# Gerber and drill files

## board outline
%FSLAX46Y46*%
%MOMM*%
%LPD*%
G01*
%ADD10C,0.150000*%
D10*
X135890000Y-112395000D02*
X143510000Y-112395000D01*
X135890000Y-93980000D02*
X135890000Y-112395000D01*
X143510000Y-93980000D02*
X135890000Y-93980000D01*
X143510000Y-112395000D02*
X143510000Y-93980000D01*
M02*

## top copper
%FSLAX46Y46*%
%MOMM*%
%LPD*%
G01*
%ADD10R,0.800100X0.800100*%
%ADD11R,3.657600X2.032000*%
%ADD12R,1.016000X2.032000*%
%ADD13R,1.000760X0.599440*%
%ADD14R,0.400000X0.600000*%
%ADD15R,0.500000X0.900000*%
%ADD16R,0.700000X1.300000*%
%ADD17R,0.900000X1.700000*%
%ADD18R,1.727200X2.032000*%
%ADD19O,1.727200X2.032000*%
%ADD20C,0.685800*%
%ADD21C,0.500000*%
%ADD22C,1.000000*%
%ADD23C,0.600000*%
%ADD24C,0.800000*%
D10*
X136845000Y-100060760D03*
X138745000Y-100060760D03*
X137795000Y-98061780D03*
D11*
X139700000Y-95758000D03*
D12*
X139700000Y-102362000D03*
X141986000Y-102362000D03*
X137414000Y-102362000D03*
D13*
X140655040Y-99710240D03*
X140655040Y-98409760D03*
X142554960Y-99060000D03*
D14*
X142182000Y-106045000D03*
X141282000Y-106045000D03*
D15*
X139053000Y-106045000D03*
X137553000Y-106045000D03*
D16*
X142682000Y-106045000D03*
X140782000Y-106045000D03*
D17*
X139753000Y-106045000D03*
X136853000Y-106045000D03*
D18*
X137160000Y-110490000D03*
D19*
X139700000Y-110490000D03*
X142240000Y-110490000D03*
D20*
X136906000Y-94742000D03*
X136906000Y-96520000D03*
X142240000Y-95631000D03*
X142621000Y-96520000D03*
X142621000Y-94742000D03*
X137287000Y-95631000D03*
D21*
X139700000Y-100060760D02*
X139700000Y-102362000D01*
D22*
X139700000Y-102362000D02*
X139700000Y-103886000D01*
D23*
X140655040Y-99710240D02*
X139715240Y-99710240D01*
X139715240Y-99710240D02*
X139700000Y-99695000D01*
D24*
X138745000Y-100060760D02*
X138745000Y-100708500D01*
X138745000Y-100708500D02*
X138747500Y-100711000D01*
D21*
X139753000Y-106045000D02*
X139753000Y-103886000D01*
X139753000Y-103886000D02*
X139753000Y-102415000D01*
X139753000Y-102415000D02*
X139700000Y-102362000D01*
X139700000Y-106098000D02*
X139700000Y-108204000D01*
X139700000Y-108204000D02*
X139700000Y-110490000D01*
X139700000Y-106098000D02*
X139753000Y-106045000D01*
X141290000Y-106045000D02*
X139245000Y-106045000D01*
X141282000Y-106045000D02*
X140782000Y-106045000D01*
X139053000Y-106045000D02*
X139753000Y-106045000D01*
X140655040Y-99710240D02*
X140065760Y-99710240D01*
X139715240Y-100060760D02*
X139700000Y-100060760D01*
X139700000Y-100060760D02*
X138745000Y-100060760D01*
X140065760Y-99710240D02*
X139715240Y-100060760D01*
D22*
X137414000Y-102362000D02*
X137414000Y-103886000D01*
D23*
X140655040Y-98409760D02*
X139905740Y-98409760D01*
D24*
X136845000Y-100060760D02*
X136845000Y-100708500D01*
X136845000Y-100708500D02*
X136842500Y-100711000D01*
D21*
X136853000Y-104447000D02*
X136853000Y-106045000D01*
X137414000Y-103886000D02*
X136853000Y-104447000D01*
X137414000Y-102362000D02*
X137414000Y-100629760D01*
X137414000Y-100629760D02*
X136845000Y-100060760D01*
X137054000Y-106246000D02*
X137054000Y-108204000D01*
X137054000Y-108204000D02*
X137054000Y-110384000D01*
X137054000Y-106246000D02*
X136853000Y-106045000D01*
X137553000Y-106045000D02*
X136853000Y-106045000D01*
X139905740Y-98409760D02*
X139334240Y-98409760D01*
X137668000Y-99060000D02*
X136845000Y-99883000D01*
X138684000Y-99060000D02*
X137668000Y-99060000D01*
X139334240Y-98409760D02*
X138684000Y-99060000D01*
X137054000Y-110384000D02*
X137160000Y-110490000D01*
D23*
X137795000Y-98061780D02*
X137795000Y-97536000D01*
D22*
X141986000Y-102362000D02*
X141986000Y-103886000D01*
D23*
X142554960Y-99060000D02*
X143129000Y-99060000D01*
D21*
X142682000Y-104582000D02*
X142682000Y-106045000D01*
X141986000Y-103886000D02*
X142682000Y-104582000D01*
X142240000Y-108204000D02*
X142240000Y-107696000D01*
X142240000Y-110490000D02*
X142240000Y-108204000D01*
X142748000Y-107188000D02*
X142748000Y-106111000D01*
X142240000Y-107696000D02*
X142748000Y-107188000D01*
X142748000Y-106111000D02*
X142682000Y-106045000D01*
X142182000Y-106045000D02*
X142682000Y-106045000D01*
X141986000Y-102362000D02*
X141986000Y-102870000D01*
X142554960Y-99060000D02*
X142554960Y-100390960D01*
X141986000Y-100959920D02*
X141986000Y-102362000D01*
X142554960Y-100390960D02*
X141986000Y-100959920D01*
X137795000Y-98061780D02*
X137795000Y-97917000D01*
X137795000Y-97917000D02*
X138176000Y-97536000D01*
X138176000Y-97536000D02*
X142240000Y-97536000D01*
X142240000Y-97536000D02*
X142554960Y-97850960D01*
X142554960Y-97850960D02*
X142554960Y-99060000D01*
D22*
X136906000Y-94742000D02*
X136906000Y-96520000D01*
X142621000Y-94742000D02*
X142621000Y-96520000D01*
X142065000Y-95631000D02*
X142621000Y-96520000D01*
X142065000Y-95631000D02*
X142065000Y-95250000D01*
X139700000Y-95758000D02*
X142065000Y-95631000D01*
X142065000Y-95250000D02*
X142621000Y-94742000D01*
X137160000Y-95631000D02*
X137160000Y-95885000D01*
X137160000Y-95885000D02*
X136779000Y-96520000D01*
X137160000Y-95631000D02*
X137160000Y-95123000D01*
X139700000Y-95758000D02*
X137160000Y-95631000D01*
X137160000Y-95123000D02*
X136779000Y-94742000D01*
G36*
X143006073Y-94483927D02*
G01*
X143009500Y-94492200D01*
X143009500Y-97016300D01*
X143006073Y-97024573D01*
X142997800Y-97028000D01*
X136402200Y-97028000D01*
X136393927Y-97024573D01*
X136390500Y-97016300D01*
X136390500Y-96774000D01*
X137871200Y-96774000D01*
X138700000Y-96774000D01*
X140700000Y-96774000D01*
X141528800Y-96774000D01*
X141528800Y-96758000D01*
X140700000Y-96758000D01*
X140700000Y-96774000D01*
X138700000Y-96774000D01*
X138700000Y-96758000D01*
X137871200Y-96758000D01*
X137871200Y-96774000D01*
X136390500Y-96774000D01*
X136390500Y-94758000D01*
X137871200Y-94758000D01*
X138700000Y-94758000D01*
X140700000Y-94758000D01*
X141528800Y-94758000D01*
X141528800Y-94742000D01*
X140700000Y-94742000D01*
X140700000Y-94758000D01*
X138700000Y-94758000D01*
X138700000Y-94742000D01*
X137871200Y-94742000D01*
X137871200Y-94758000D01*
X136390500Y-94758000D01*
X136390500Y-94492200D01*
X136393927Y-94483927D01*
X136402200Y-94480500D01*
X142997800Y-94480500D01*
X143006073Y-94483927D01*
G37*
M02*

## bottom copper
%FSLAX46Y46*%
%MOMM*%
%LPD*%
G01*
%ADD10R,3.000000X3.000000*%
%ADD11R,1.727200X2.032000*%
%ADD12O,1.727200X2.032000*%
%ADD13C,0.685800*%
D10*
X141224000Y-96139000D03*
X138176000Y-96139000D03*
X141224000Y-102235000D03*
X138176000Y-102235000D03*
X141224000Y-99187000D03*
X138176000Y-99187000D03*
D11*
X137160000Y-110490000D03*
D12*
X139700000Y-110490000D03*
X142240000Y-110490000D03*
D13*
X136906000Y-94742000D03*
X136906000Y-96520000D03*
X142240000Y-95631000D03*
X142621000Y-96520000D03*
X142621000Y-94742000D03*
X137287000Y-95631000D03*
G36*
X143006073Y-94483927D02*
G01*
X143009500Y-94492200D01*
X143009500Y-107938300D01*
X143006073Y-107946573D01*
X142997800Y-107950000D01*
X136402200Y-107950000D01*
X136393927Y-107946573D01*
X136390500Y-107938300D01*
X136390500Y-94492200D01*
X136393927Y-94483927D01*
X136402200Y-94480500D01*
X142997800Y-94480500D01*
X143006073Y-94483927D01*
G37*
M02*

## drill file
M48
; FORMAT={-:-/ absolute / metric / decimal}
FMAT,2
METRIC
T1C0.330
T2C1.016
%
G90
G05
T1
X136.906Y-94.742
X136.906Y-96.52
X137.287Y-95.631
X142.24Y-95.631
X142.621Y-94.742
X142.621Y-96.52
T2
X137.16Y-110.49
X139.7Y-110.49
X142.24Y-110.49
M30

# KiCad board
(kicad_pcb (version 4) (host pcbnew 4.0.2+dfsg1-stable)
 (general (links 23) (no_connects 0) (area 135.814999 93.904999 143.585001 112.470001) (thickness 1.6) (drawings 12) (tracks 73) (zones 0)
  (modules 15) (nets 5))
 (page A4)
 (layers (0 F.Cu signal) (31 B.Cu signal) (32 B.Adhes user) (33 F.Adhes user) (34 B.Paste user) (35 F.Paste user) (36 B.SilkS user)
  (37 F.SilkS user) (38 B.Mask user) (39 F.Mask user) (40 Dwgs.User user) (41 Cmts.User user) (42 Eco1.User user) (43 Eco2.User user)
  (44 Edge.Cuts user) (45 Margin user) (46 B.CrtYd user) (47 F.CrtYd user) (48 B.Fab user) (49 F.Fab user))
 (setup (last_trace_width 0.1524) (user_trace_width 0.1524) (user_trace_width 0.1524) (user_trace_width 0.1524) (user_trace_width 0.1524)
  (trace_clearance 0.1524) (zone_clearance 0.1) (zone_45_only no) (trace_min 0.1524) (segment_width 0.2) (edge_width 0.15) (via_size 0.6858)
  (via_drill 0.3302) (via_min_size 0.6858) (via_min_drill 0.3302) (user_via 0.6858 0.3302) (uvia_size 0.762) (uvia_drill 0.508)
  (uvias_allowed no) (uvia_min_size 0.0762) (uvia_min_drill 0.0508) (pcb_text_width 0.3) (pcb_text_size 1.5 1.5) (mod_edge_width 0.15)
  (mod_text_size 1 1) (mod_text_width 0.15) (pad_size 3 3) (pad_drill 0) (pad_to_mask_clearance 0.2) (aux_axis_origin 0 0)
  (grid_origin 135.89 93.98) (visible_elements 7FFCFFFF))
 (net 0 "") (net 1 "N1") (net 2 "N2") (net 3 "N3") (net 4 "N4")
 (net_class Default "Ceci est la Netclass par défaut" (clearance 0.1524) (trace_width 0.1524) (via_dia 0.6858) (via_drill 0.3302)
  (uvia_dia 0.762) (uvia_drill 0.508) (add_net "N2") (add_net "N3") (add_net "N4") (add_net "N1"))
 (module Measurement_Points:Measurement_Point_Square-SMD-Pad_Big (layer B.Cu) (at 141.224 96.139)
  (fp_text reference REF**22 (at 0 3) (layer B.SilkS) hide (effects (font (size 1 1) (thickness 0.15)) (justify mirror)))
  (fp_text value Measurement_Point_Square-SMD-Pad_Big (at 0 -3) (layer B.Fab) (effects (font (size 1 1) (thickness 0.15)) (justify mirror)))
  (pad 1 smd rect (at 0 0) (size 3 3) (layers B.Cu B.Mask) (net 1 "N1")))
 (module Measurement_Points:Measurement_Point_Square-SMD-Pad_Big (layer B.Cu) (at 138.176 96.139)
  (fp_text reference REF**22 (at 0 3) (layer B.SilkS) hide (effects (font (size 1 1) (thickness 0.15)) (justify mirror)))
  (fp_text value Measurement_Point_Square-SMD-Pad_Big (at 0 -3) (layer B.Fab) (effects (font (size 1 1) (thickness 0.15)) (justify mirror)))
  (pad 1 smd rect (at 0 0) (size 3 3) (layers B.Cu B.Mask) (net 1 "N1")))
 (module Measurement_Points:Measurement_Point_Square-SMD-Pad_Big (layer B.Cu) (at 141.224 102.235)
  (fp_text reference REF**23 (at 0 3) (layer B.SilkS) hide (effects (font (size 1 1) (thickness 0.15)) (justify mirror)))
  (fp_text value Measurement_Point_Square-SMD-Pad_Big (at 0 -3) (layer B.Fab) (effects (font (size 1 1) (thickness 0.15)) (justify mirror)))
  (pad 1 smd rect (at 0 0) (size 3 3) (layers B.Cu B.Mask) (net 1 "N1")))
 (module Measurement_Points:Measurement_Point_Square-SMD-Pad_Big (layer B.Cu) (at 138.176 102.235)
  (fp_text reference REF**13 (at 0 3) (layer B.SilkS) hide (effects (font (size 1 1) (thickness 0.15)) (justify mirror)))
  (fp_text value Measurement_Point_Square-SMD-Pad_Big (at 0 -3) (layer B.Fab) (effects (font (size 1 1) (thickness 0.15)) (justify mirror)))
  (pad 1 smd rect (at 0 0) (size 3 3) (layers B.Cu B.Mask) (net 1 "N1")))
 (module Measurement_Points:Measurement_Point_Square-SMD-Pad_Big (layer B.Cu) (at 141.224 99.187)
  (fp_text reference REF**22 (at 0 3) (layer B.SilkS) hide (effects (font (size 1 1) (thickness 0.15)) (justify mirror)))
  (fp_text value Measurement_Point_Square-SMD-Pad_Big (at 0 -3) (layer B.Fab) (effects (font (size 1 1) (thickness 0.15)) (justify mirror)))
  (pad 1 smd rect (at 0 0) (size 3 3) (layers B.Cu B.Mask) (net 1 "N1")))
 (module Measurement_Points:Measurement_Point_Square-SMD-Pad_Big (layer B.Cu) (at 138.176 99.187) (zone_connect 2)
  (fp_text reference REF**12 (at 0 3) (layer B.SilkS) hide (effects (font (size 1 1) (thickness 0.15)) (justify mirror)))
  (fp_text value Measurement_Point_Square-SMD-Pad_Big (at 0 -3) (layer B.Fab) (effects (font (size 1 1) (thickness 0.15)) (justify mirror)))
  (pad 1 smd rect (at 0 0) (size 3 3) (layers B.Cu B.Mask) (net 1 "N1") (zone_connect 2)))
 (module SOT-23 (layer F.Cu) (at 137.795 99.06)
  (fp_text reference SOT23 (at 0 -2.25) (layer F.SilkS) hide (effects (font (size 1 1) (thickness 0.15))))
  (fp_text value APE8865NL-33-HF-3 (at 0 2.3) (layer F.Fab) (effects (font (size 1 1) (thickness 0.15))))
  (pad 1 smd rect (at -0.95 1.00076) (size 0.8001 0.8001) (layers F.Cu F.Paste F.Mask) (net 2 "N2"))
  (pad 2 smd rect (at 0.95 1.00076) (size 0.8001 0.8001) (layers F.Cu F.Paste F.Mask) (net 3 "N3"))
  (pad 3 smd rect (at 0 -0.99822) (size 0.8001 0.8001) (layers F.Cu F.Paste F.Mask) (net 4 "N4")))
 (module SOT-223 (layer F.Cu) (at 139.7 99.06)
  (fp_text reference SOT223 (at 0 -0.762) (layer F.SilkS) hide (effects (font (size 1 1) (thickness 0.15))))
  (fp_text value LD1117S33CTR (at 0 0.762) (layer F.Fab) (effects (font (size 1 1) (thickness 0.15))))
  (pad 4 smd rect (at 0 -3.302) (size 3.6576 2.032) (layers F.Cu F.Paste F.Mask) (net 1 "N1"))
  (pad 2 smd rect (at 0 3.302) (size 1.016 2.032) (layers F.Cu F.Paste F.Mask) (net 3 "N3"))
  (pad 3 smd rect (at 2.286 3.302) (size 1.016 2.032) (layers F.Cu F.Paste F.Mask) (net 4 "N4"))
  (pad 1 smd rect (at -2.286 3.302) (size 1.016 2.032) (layers F.Cu F.Paste F.Mask) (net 2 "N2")))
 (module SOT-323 (layer F.Cu) (at 141.605 99.06 90)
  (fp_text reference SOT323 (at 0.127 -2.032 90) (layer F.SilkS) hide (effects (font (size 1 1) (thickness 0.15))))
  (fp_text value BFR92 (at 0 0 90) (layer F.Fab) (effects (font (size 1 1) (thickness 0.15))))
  (pad 2 smd rect (at -0.65024 -0.94996 90) (size 0.59944 1.00076) (layers F.Cu F.Paste F.Mask) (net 3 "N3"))
  (pad 1 smd rect (at 0.65024 -0.94996 90) (size 0.59944 1.00076) (layers F.Cu F.Paste F.Mask) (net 2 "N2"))
  (pad 3 smd rect (at 0 0.94996 90) (size 0.59944 1.00076) (layers F.Cu F.Paste F.Mask) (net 4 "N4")))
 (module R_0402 (layer F.Cu) (at 141.732 106.045 180)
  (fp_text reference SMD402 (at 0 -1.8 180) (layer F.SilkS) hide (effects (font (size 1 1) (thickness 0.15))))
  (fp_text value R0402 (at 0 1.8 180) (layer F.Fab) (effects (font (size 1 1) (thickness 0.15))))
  (pad 1 smd rect (at -0.45 0 180) (size 0.4 0.6) (layers F.Cu F.Paste F.Mask) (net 4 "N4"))
  (pad 2 smd rect (at 0.45 0 180) (size 0.4 0.6) (layers F.Cu F.Paste F.Mask) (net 3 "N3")))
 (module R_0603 (layer F.Cu) (at 138.303 106.045 180)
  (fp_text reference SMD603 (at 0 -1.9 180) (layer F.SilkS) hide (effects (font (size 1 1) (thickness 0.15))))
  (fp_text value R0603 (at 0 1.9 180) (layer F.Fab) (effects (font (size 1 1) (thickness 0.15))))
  (pad 1 smd rect (at -0.75 0 180) (size 0.5 0.9) (layers F.Cu F.Paste F.Mask) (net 3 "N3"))
  (pad 2 smd rect (at 0.75 0 180) (size 0.5 0.9) (layers F.Cu F.Paste F.Mask) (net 2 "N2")))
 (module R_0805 (layer F.Cu) (at 141.732 106.045 180)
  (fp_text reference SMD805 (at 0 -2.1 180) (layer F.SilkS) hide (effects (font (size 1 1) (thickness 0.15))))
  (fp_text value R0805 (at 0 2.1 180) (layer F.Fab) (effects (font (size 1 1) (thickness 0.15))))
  (pad 1 smd rect (at -0.95 0 180) (size 0.7 1.3) (layers F.Cu F.Paste F.Mask) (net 4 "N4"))
  (pad 2 smd rect (at 0.95 0 180) (size 0.7 1.3) (layers F.Cu F.Paste F.Mask) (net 3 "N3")))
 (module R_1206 (layer F.Cu) (at 138.303 106.045 180)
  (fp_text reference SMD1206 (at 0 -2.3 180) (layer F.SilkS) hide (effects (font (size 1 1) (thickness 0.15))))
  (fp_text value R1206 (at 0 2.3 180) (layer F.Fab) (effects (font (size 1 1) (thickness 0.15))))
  (pad 1 smd rect (at -1.45 0 180) (size 0.9 1.7) (layers F.Cu F.Paste F.Mask) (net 3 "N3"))
  (pad 2 smd rect (at 1.45 0 180) (size 0.9 1.7) (layers F.Cu F.Paste F.Mask) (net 2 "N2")))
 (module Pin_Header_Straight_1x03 (layer F.Cu) (at 137.16 110.49 90)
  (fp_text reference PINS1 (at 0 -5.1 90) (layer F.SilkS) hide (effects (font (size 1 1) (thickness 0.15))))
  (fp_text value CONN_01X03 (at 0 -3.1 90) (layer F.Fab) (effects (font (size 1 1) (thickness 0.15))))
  (pad 1 thru_hole rect (at 0 0 90) (size 2.032 1.7272) (drill 1.016) (layers *.Cu *.Mask F.SilkS) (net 2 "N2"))
  (pad 2 thru_hole oval (at 0 2.54 90) (size 2.032 1.7272) (drill 1.016) (layers *.Cu *.Mask F.SilkS) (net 3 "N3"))
  (pad 3 thru_hole oval (at 0 5.08 90) (size 2.032 1.7272) (drill 1.016) (layers *.Cu *.Mask F.SilkS) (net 4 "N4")))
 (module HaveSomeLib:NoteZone (layer B.Cu) (at 139.7 108.204)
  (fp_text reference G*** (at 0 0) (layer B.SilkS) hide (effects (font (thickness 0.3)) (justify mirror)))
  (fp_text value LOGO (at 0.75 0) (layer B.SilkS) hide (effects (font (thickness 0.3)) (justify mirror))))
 (gr_line (start 135.89 112.395) (end 143.51 112.395) (angle 90) (layer Edge.Cuts) (width 0.15))
 (gr_line (start 135.89 93.98) (end 135.89 112.395) (angle 90) (layer Edge.Cuts) (width 0.15))
 (gr_line (start 143.51 93.98) (end 135.89 93.98) (angle 90) (layer Edge.Cuts) (width 0.15))
 (gr_line (start 143.51 112.395) (end 143.51 93.98) (angle 90) (layer Edge.Cuts) (width 0.15))
 (segment (start 139.7 100.06076) (end 139.7 102.362) (width 0.5) (layer F.Cu) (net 3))
 (segment (start 139.7 102.362) (end 139.7 103.886) (width 1) (layer F.Cu) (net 3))
 (segment (start 140.65504 99.71024) (end 139.71524 99.71024) (width 0.6) (layer F.Cu) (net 3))
 (segment (start 139.71524 99.71024) (end 139.7 99.695) (width 0.6) (layer F.Cu) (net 3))
 (segment (start 138.745 100.06076) (end 138.745 100.7085) (width 0.8) (layer F.Cu) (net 3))
 (segment (start 138.745 100.7085) (end 138.7475 100.711) (width 0.8) (layer F.Cu) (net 3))
 (segment (start 139.753 106.045) (end 139.753 103.886) (width 0.5) (layer F.Cu) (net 3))
 (segment (start 139.753 103.886) (end 139.753 102.415) (width 0.5) (layer F.Cu) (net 3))
 (segment (start 139.753 102.415) (end 139.7 102.362) (width 0.5) (layer F.Cu) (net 3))
 (segment (start 139.7 106.098) (end 139.7 108.204) (width 0.5) (layer F.Cu) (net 3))
 (segment (start 139.7 108.204) (end 139.7 110.49) (width 0.5) (layer F.Cu) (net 3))
 (segment (start 139.7 106.098) (end 139.753 106.045) (width 0.5) (layer F.Cu) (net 3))
 (segment (start 141.29 106.045) (end 139.245 106.045) (width 0.5) (layer F.Cu) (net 3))
 (segment (start 141.282 106.045) (end 140.782 106.045) (width 0.5) (layer F.Cu) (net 3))
 (segment (start 139.053 106.045) (end 139.753 106.045) (width 0.5) (layer F.Cu) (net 3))
 (segment (start 140.65504 99.71024) (end 140.06576 99.71024) (width 0.5) (layer F.Cu) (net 3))
 (segment (start 139.71524 100.06076) (end 139.7 100.06076) (width 0.5) (layer F.Cu) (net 3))
 (segment (start 139.7 100.06076) (end 138.745 100.06076) (width 0.5) (layer F.Cu) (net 3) (status 20))
 (segment (start 140.06576 99.71024) (end 139.71524 100.06076) (width 0.5) (layer F.Cu) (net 3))
 (segment (start 137.414 102.362) (end 137.414 103.886) (width 1) (layer F.Cu) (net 2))
 (segment (start 140.65504 98.40976) (end 139.90574 98.40976) (width 0.6) (layer F.Cu) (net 2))
 (segment (start 136.845 100.06076) (end 136.845 100.7085) (width 0.8) (layer F.Cu) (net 2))
 (segment (start 136.845 100.7085) (end 136.8425 100.711) (width 0.8) (layer F.Cu) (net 2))
 (segment (start 136.853 104.447) (end 136.853 106.045) (width 0.5) (layer F.Cu) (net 2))
 (segment (start 137.414 103.886) (end 136.853 104.447) (width 0.5) (layer F.Cu) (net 2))
 (segment (start 137.414 102.362) (end 137.414 100.62976) (width 0.5) (layer F.Cu) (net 2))
 (segment (start 137.414 100.62976) (end 136.845 100.06076) (width 0.5) (layer F.Cu) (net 2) (status 20))
 (segment (start 137.054 106.246) (end 137.054 108.204) (width 0.5) (layer F.Cu) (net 2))
 (segment (start 137.054 108.204) (end 137.054 110.384) (width 0.5) (layer F.Cu) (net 2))
 (segment (start 137.054 106.246) (end 136.853 106.045) (width 0.5) (layer F.Cu) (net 2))
 (segment (start 137.553 106.045) (end 136.853 106.045) (width 0.5) (layer F.Cu) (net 2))
 (segment (start 139.90574 98.40976) (end 139.33424 98.40976) (width 0.5) (layer F.Cu) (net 2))
 (segment (start 137.668 99.06) (end 136.845 99.883) (width 0.5) (layer F.Cu) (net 2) (status 20))
 (segment (start 138.684 99.06) (end 137.668 99.06) (width 0.5) (layer F.Cu) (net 2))
 (segment (start 139.33424 98.40976) (end 138.684 99.06) (width 0.5) (layer F.Cu) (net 2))
 (segment (start 137.054 110.384) (end 137.16 110.49) (width 0.5) (layer F.Cu) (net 2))
 (segment (start 137.795 98.06178) (end 137.795 97.536) (width 0.6) (layer F.Cu) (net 4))
 (segment (start 141.986 102.362) (end 141.986 103.886) (width 1) (layer F.Cu) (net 4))
 (segment (start 142.55496 99.06) (end 143.129 99.06) (width 0.6) (layer F.Cu) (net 4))
 (segment (start 142.682 104.582) (end 142.682 106.045) (width 0.5) (layer F.Cu) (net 4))
 (segment (start 141.986 103.886) (end 142.682 104.582) (width 0.5) (layer F.Cu) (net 4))
 (segment (start 142.24 108.204) (end 142.24 107.696) (width 0.5) (layer F.Cu) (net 4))
 (segment (start 142.24 110.49) (end 142.24 108.204) (width 0.5) (layer F.Cu) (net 4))
 (segment (start 142.748 107.188) (end 142.748 106.111) (width 0.5) (layer F.Cu) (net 4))
 (segment (start 142.24 107.696) (end 142.748 107.188) (width 0.5) (layer F.Cu) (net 4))
 (segment (start 142.748 106.111) (end 142.682 106.045) (width 0.5) (layer F.Cu) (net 4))
 (segment (start 142.182 106.045) (end 142.682 106.045) (width 0.5) (layer F.Cu) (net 4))
 (segment (start 141.986 102.362) (end 141.986 102.87) (width 0.5) (layer F.Cu) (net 4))
 (segment (start 142.55496 99.06) (end 142.55496 100.39096) (width 0.5) (layer F.Cu) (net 4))
 (segment (start 141.986 100.95992) (end 141.986 102.362) (width 0.5) (layer F.Cu) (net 4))
 (segment (start 142.55496 100.39096) (end 141.986 100.95992) (width 0.5) (layer F.Cu) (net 4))
 (segment (start 137.795 98.06178) (end 137.795 97.917) (width 0.5) (layer F.Cu) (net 4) (status 30))
 (segment (start 137.795 97.917) (end 138.176 97.536) (width 0.5) (layer F.Cu) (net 4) (status 10))
 (segment (start 138.176 97.536) (end 142.24 97.536) (width 0.5) (layer F.Cu) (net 4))
 (segment (start 142.24 97.536) (end 142.55496 97.85096) (width 0.5) (layer F.Cu) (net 4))
 (segment (start 142.55496 97.85096) (end 142.55496 99.06) (width 0.5) (layer F.Cu) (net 4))
 (segment (start 136.906 94.742) (end 136.906 96.52) (width 1) (layer F.Cu) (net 1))
 (via (at 136.906 94.742) (size 0.6858) (drill 0.3302) (layers F.Cu B.Cu) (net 1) (status 30))
 (via (at 136.906 96.52) (size 0.6858) (drill 0.3302) (layers F.Cu B.Cu) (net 1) (status 30))
 (segment (start 142.621 94.742) (end 142.621 96.52) (width 1) (layer F.Cu) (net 1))
 (segment (start 142.065 95.631) (end 142.621 96.52) (width 1) (layer F.Cu) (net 1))
 (via (at 142.24 95.631) (size 0.6858) (drill 0.3302) (layers F.Cu B.Cu) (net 1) (status 30))
 (via (at 142.621 96.52) (size 0.6858) (drill 0.3302) (layers F.Cu B.Cu) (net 1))
 (segment (start 142.065 95.631) (end 142.065 95.25) (width 1) (layer F.Cu) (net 1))
 (segment (start 139.7 95.758) (end 142.065 95.631) (width 1) (layer F.Cu) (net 1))
 (via (at 142.621 94.742) (size 0.6858) (drill 0.3302) (layers F.Cu B.Cu) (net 1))
 (segment (start 142.065 95.25) (end 142.621 94.742) (width 1) (layer F.Cu) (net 1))
 (segment (start 137.16 95.631) (end 137.16 95.885) (width 1) (layer F.Cu) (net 1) (status 30))
 (via (at 137.287 95.631) (size 0.6858) (drill 0.3302) (layers F.Cu B.Cu) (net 1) (status 30))
 (segment (start 137.16 95.885) (end 136.779 96.52) (width 1) (layer F.Cu) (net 1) (status 30))
 (segment (start 137.16 95.631) (end 137.16 95.123) (width 1) (layer F.Cu) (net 1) (status 30))
 (segment (start 139.7 95.758) (end 137.16 95.631) (width 1) (layer F.Cu) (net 1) (status 20))
 (segment (start 137.16 95.123) (end 136.779 94.742) (width 1) (layer F.Cu) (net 1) (status 30))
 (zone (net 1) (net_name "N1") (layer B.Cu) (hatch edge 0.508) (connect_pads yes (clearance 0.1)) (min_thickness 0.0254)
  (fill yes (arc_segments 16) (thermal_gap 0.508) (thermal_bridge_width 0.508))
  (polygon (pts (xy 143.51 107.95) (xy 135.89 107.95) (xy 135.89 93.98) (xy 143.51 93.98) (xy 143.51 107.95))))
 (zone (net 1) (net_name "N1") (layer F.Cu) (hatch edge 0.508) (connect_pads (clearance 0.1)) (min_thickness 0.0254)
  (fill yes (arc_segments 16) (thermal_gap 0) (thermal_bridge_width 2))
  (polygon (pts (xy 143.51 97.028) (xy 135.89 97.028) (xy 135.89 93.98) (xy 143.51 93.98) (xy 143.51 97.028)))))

